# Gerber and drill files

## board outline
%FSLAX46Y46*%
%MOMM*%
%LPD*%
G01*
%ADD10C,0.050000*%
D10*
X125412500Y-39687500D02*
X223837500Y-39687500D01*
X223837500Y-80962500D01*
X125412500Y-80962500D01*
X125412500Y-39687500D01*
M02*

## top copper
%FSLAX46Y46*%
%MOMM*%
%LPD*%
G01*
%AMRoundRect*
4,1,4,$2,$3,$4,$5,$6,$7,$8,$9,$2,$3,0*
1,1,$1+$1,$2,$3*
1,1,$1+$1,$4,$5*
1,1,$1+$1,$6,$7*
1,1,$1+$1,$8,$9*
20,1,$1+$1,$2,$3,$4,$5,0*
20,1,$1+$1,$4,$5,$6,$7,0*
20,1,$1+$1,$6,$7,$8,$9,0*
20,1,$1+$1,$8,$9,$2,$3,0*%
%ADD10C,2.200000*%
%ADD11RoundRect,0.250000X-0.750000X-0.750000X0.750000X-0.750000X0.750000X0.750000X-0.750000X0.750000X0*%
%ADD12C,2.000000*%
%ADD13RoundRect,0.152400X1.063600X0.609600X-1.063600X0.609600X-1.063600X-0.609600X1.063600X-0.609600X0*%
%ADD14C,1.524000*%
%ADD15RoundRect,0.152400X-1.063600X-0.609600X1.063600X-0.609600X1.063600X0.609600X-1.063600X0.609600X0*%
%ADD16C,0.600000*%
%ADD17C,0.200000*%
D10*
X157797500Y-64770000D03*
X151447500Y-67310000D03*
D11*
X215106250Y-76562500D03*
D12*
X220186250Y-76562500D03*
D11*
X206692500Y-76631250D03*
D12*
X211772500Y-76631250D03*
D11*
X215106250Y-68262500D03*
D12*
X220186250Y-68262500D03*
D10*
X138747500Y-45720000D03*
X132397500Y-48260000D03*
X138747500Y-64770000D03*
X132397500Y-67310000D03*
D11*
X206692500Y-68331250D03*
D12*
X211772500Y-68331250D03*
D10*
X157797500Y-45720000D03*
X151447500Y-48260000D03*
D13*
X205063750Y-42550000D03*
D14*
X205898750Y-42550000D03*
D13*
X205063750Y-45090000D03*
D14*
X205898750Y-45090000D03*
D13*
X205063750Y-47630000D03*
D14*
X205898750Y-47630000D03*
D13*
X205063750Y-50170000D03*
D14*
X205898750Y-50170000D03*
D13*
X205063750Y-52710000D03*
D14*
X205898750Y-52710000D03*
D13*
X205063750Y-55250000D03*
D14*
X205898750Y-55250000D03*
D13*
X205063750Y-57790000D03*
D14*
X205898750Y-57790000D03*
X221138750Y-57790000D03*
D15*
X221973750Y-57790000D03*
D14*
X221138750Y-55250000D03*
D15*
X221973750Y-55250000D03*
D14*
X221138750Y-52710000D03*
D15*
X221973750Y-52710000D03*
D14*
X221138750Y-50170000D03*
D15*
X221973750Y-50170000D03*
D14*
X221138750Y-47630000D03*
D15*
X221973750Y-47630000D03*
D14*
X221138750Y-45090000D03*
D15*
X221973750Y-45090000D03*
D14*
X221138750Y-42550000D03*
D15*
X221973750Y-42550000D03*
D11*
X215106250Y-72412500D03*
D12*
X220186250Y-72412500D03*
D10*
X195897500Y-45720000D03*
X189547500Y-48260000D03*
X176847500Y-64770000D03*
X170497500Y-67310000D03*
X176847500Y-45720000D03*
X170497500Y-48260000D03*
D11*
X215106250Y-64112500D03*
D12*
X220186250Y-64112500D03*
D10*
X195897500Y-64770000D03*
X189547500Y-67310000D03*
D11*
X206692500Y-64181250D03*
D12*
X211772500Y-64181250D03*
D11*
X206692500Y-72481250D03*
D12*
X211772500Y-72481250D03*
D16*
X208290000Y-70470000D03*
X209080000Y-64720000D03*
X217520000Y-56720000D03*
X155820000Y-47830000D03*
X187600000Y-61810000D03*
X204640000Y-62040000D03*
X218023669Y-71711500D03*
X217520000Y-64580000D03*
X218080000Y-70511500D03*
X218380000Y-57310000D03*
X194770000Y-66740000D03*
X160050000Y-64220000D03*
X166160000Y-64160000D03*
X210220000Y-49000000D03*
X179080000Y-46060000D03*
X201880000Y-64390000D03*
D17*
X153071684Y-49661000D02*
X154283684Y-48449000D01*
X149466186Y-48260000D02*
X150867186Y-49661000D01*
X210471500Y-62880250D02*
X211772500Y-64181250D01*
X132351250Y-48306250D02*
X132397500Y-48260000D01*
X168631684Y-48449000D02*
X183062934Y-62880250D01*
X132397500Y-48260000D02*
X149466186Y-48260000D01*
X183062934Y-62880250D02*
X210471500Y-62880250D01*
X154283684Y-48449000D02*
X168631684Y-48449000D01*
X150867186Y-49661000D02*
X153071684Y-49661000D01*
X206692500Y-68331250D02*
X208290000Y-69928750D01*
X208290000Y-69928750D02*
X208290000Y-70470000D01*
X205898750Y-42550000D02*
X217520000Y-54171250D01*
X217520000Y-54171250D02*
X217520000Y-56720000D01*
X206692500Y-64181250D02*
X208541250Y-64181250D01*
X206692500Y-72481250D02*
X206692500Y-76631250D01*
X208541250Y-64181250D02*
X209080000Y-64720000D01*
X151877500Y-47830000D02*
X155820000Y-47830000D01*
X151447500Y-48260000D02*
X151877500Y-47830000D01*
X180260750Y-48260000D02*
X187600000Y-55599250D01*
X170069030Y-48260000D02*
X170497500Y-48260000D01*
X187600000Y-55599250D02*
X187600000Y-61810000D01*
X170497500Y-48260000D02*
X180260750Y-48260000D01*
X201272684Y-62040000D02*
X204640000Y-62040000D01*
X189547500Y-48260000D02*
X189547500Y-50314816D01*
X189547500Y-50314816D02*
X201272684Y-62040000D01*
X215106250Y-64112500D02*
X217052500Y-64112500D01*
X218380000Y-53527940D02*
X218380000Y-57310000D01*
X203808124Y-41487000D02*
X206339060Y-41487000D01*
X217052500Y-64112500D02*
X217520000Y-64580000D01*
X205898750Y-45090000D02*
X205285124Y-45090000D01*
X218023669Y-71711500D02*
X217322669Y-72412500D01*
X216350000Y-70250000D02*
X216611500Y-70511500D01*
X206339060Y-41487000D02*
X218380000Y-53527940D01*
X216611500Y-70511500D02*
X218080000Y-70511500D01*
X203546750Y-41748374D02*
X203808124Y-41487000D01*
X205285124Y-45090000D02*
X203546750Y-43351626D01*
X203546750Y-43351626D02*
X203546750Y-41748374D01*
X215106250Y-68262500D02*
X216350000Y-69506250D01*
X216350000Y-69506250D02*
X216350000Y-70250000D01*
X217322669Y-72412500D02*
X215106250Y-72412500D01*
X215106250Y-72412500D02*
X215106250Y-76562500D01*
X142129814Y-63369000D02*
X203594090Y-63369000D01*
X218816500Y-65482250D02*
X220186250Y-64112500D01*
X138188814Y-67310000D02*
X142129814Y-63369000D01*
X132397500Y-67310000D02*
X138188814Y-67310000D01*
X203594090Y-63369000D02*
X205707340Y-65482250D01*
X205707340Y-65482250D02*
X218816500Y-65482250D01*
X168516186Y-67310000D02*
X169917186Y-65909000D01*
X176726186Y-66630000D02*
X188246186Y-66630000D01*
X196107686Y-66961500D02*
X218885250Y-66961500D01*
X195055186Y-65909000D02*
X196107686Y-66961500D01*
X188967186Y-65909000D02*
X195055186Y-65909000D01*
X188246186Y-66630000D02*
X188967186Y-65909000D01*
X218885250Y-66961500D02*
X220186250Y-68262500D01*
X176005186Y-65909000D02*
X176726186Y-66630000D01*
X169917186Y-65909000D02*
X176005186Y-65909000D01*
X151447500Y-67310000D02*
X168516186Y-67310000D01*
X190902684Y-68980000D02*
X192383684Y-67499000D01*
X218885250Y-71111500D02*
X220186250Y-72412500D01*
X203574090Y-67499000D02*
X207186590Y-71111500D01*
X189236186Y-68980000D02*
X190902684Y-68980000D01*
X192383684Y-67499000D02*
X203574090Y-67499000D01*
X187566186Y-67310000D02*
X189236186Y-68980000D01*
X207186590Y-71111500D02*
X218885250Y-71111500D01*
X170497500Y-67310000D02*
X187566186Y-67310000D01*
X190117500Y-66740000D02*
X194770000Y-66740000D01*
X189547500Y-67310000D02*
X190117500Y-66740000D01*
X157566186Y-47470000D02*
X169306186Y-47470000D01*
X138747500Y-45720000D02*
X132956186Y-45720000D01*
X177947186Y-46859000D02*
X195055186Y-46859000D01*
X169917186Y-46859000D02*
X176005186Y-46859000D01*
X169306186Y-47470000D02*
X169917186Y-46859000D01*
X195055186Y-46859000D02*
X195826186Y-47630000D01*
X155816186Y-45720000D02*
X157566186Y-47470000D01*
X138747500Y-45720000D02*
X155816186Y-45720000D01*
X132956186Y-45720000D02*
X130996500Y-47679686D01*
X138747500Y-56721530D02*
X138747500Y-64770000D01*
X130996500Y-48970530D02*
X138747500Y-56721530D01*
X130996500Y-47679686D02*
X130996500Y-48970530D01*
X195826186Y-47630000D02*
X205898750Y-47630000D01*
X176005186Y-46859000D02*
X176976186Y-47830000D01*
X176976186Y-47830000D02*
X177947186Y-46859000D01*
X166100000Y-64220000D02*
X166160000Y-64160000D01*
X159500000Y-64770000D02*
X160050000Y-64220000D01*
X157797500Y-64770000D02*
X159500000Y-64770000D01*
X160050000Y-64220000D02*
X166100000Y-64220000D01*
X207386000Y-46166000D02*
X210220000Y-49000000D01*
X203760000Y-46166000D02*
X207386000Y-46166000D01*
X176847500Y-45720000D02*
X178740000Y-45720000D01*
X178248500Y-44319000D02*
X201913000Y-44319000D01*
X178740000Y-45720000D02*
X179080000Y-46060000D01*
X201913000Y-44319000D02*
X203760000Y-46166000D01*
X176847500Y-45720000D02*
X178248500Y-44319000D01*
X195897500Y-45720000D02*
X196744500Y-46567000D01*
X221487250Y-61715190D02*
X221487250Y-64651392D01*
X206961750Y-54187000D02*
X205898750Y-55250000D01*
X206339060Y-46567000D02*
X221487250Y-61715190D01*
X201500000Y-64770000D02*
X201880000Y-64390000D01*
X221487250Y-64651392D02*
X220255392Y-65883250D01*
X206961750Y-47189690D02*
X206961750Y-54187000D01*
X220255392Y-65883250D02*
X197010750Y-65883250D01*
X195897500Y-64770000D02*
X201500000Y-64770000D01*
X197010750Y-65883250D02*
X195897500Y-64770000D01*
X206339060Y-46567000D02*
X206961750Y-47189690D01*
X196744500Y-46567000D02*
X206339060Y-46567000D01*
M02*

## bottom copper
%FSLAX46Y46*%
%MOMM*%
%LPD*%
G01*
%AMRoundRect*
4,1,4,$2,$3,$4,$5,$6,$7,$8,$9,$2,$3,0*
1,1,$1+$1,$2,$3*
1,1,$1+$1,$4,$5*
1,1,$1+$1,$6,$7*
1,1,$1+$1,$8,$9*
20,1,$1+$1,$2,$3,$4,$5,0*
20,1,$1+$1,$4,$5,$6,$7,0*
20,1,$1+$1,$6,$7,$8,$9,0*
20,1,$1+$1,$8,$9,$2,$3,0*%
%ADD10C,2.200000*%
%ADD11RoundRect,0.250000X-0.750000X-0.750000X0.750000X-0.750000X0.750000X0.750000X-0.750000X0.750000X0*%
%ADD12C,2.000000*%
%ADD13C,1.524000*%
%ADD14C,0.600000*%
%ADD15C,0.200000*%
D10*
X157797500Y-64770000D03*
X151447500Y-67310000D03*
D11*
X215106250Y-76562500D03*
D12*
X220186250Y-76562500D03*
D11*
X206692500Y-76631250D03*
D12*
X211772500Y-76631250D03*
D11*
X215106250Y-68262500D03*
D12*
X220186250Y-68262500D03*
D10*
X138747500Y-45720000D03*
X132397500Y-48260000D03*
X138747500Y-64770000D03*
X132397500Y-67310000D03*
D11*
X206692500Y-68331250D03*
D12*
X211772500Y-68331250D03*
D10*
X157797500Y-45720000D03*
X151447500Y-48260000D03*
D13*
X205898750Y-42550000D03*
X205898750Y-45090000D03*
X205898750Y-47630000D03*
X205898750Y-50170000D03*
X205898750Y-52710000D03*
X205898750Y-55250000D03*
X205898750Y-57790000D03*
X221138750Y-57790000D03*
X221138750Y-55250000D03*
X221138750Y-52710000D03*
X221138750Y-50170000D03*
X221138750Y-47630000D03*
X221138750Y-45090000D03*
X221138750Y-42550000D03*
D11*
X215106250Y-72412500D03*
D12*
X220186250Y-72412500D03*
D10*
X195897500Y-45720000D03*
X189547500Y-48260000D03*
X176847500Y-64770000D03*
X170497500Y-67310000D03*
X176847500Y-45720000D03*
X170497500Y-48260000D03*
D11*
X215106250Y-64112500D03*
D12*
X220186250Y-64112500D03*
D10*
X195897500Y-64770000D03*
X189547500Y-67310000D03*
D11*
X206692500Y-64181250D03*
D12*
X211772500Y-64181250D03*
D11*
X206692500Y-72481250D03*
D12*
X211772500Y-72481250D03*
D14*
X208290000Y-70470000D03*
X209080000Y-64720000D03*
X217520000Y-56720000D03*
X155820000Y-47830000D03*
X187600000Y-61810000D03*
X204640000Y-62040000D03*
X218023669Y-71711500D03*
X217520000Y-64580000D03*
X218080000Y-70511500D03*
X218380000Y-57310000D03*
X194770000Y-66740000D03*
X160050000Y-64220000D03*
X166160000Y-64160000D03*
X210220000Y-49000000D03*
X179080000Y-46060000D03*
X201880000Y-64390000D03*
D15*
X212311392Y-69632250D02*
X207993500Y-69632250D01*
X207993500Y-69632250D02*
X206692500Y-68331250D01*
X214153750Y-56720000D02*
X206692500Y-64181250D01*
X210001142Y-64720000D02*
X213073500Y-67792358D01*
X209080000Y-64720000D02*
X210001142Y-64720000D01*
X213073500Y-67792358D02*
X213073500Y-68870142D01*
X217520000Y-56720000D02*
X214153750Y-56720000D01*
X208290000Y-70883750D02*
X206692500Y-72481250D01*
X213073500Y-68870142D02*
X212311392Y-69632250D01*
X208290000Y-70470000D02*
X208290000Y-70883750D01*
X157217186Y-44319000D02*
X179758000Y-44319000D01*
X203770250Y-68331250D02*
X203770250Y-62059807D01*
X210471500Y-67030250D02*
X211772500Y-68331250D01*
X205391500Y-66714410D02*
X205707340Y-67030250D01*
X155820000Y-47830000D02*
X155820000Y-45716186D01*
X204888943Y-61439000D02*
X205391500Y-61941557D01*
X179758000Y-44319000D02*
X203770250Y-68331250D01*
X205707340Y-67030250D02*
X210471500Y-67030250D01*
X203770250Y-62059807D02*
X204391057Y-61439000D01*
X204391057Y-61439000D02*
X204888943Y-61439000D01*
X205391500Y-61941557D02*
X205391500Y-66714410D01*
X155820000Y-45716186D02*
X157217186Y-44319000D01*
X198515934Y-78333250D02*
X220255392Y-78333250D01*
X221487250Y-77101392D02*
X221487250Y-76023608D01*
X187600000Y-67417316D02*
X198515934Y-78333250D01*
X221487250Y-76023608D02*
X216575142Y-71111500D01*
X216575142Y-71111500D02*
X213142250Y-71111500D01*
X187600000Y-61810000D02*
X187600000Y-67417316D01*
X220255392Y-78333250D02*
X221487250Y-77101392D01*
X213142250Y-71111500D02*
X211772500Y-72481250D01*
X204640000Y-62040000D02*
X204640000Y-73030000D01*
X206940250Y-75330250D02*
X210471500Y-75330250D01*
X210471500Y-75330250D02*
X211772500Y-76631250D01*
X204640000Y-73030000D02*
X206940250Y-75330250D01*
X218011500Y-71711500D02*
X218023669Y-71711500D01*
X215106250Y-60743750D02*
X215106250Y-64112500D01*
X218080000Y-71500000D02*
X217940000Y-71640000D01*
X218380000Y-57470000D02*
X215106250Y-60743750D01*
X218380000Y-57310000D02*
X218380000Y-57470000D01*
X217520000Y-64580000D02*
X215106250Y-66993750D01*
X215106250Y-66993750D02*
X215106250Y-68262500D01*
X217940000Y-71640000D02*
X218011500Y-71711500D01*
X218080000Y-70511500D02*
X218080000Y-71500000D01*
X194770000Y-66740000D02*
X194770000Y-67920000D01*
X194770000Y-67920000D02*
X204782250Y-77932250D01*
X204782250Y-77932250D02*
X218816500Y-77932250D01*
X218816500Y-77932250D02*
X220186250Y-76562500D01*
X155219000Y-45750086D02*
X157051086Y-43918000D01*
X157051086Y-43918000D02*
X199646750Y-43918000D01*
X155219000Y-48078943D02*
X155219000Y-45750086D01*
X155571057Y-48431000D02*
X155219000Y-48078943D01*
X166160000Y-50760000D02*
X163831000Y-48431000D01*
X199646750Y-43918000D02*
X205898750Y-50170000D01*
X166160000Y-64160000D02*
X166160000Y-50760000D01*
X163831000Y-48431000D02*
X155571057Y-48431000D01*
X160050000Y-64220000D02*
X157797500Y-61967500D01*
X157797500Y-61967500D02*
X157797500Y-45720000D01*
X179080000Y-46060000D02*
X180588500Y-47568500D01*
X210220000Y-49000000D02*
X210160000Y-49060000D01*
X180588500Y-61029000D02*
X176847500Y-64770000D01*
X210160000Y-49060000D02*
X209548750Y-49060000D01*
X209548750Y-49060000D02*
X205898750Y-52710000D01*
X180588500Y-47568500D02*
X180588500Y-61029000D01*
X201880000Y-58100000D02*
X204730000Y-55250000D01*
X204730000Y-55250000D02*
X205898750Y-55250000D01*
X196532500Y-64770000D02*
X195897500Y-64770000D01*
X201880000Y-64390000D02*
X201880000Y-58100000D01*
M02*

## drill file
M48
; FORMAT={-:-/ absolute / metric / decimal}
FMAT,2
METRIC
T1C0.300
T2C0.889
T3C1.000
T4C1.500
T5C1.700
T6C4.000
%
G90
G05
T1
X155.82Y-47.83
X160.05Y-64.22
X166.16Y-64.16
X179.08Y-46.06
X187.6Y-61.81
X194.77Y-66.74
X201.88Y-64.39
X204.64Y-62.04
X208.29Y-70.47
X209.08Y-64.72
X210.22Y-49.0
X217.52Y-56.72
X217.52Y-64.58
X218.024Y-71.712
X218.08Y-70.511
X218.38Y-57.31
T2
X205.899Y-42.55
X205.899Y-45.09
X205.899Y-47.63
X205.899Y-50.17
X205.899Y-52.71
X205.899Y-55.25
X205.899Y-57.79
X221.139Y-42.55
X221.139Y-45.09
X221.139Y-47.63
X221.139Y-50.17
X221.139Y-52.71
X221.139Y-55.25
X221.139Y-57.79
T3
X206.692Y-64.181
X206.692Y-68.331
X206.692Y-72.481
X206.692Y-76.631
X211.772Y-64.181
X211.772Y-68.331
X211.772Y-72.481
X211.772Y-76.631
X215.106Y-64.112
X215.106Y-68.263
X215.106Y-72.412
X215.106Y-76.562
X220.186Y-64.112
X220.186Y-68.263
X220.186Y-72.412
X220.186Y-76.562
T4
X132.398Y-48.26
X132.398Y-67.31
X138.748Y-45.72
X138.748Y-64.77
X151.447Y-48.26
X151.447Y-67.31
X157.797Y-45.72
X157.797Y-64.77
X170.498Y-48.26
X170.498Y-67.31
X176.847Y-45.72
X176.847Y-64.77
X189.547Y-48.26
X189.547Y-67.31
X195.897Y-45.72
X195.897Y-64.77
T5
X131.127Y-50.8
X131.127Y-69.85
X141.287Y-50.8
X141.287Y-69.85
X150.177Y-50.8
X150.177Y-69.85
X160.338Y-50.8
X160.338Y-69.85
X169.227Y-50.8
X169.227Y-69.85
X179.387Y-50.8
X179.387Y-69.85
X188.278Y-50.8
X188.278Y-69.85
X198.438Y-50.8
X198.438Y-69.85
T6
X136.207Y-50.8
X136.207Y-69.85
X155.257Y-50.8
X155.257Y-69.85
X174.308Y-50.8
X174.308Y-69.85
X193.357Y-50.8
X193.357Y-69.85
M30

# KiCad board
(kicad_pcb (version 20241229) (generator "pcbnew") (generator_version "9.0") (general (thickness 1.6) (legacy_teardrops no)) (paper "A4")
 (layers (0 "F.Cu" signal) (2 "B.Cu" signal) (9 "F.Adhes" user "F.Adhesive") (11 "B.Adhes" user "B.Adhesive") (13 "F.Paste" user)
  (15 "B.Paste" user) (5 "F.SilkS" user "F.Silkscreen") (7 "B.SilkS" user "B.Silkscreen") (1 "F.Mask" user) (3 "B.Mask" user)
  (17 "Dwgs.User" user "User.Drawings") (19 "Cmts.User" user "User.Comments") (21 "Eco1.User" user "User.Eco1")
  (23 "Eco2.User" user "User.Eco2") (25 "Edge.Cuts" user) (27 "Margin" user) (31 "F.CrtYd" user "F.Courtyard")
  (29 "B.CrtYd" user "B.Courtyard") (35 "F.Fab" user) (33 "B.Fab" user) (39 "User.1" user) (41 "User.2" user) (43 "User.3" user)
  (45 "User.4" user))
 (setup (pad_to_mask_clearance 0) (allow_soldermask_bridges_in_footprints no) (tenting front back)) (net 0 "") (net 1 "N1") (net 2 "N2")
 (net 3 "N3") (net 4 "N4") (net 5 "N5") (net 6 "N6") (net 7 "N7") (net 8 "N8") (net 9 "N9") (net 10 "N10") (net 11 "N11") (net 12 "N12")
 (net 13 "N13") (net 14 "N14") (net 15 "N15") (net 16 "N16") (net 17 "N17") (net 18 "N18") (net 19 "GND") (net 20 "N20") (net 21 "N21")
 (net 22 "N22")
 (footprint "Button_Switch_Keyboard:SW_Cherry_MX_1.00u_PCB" (layer "F.Cu") (at 157.7975 64.77)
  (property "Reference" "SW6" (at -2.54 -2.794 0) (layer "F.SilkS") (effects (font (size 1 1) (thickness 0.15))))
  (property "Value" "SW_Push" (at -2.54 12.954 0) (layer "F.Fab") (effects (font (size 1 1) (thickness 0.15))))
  (pad "" np_thru_hole circle (at -7.62 5.08) (size 1.7 1.7) (drill 1.7) (layers "*.Cu" "*.Mask"))
  (pad "" np_thru_hole circle (at -2.54 5.08) (size 4 4) (drill 4) (layers "*.Cu" "*.Mask"))
  (pad "" np_thru_hole circle (at 2.54 5.08) (size 1.7 1.7) (drill 1.7) (layers "*.Cu" "*.Mask"))
  (pad "1" thru_hole circle (at 0 0) (size 2.2 2.2) (drill 1.5) (layers "*.Cu" "*.Mask") (remove_unused_layers no) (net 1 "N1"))
  (pad "2" thru_hole circle (at -6.35 2.54) (size 2.2 2.2) (drill 1.5) (layers "*.Cu" "*.Mask") (remove_unused_layers no) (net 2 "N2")))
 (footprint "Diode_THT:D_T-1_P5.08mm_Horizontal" (layer "F.Cu") (at 215.10625 76.5625)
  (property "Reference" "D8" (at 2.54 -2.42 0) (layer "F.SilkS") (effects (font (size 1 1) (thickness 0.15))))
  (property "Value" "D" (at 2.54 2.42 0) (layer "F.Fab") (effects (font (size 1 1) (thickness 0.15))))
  (pad "1" thru_hole roundrect (at 0 0) (size 2 2) (drill 1) (layers "*.Cu" "*.Mask") (remove_unused_layers no) (roundrect_rratio 0.125)
   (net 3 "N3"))
  (pad "2" thru_hole circle (at 5.08 0) (size 2 2) (drill 1) (layers "*.Cu" "*.Mask") (remove_unused_layers no) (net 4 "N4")))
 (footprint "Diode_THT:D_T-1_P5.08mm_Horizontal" (layer "F.Cu") (at 206.6925 76.63125)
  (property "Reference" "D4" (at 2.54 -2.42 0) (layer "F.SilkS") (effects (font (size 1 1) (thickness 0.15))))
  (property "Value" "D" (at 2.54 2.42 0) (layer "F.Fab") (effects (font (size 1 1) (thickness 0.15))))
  (pad "1" thru_hole roundrect (at 0 0) (size 2 2) (drill 1) (layers "*.Cu" "*.Mask") (remove_unused_layers no) (roundrect_rratio 0.125)
   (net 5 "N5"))
  (pad "2" thru_hole circle (at 5.08 0) (size 2 2) (drill 1) (layers "*.Cu" "*.Mask") (remove_unused_layers no) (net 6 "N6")))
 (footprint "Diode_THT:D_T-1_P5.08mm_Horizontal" (layer "F.Cu") (at 215.10625 68.2625)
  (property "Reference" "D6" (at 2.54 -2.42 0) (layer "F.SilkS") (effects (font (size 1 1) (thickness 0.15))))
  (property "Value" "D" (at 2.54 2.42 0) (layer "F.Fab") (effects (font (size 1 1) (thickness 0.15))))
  (pad "1" thru_hole roundrect (at 0 0) (size 2 2) (drill 1) (layers "*.Cu" "*.Mask") (remove_unused_layers no) (roundrect_rratio 0.125)
   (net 3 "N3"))
  (pad "2" thru_hole circle (at 5.08 0) (size 2 2) (drill 1) (layers "*.Cu" "*.Mask") (remove_unused_layers no) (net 2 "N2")))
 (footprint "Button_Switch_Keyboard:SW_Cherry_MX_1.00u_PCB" (layer "F.Cu") (at 138.7475 45.72)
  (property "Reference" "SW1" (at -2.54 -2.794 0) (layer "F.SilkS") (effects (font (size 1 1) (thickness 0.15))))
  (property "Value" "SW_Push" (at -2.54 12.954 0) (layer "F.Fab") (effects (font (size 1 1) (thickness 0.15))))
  (pad "" np_thru_hole circle (at -7.62 5.08) (size 1.7 1.7) (drill 1.7) (layers "*.Cu" "*.Mask"))
  (pad "" np_thru_hole circle (at -2.54 5.08) (size 4 4) (drill 4) (layers "*.Cu" "*.Mask"))
  (pad "" np_thru_hole circle (at 2.54 5.08) (size 1.7 1.7) (drill 1.7) (layers "*.Cu" "*.Mask"))
  (pad "1" thru_hole circle (at 0 0) (size 2.2 2.2) (drill 1.5) (layers "*.Cu" "*.Mask") (remove_unused_layers no) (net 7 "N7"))
  (pad "2" thru_hole circle (at -6.35 2.54) (size 2.2 2.2) (drill 1.5) (layers "*.Cu" "*.Mask") (remove_unused_layers no) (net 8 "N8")))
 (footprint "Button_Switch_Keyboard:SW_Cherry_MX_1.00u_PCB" (layer "F.Cu") (at 138.7475 64.77)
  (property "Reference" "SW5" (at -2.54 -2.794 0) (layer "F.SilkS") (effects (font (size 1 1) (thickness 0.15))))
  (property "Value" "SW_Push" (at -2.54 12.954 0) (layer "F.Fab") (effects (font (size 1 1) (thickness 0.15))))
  (pad "" np_thru_hole circle (at -7.62 5.08) (size 1.7 1.7) (drill 1.7) (layers "*.Cu" "*.Mask"))
  (pad "" np_thru_hole circle (at -2.54 5.08) (size 4 4) (drill 4) (layers "*.Cu" "*.Mask"))
  (pad "" np_thru_hole circle (at 2.54 5.08) (size 1.7 1.7) (drill 1.7) (layers "*.Cu" "*.Mask"))
  (pad "1" thru_hole circle (at 0 0) (size 2.2 2.2) (drill 1.5) (layers "*.Cu" "*.Mask") (remove_unused_layers no) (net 7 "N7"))
  (pad "2" thru_hole circle (at -6.35 2.54) (size 2.2 2.2) (drill 1.5) (layers "*.Cu" "*.Mask") (remove_unused_layers no) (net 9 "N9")))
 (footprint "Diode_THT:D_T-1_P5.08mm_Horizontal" (layer "F.Cu") (at 206.6925 68.33125)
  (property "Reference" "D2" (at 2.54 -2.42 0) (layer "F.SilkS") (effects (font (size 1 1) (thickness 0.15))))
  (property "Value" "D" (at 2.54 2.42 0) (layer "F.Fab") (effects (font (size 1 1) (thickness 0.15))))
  (pad "1" thru_hole roundrect (at 0 0) (size 2 2) (drill 1) (layers "*.Cu" "*.Mask") (remove_unused_layers no) (roundrect_rratio 0.125)
   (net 5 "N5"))
  (pad "2" thru_hole circle (at 5.08 0) (size 2 2) (drill 1) (layers "*.Cu" "*.Mask") (remove_unused_layers no) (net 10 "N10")))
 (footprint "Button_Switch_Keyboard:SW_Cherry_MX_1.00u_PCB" (layer "F.Cu") (at 157.7975 45.72)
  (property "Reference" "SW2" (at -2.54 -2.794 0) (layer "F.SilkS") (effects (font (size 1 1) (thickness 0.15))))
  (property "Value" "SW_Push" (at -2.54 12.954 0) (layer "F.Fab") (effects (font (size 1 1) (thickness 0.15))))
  (pad "" np_thru_hole circle (at -7.62 5.08) (size 1.7 1.7) (drill 1.7) (layers "*.Cu" "*.Mask"))
  (pad "" np_thru_hole circle (at -2.54 5.08) (size 4 4) (drill 4) (layers "*.Cu" "*.Mask"))
  (pad "" np_thru_hole circle (at 2.54 5.08) (size 1.7 1.7) (drill 1.7) (layers "*.Cu" "*.Mask"))
  (pad "1" thru_hole circle (at 0 0) (size 2.2 2.2) (drill 1.5) (layers "*.Cu" "*.Mask") (remove_unused_layers no) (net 1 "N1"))
  (pad "2" thru_hole circle (at -6.35 2.54) (size 2.2 2.2) (drill 1.5) (layers "*.Cu" "*.Mask") (remove_unused_layers no) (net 10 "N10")))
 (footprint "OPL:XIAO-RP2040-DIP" (layer "F.Cu") (at 213.51875 50.17)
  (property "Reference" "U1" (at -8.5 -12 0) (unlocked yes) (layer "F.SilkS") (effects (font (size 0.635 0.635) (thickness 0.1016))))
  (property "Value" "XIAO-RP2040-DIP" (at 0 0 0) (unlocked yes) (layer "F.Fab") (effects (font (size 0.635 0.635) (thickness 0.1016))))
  (pad "1" smd roundrect (at -8.455 -7.62 180) (size 2.432 1.524) (layers "F.Cu" "F.Mask") (roundrect_rratio 0.1) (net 5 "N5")
   (thermal_bridge_angle 45))
  (pad "1" thru_hole circle (at -7.62 -7.62 180) (size 1.524 1.524) (drill 0.889) (layers "*.Cu" "*.Mask") (remove_unused_layers no)
   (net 5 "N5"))
  (pad "2" smd roundrect (at -8.455 -5.08 180) (size 2.432 1.524) (layers "F.Cu" "F.Mask") (roundrect_rratio 0.1) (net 3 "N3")
   (thermal_bridge_angle 45))
  (pad "2" thru_hole circle (at -7.62 -5.08 180) (size 1.524 1.524) (drill 0.889) (layers "*.Cu" "*.Mask") (remove_unused_layers no)
   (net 3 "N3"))
  (pad "3" smd roundrect (at -8.455 -2.54 180) (size 2.432 1.524) (layers "F.Cu" "F.Mask") (roundrect_rratio 0.1) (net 7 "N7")
   (thermal_bridge_angle 45))
  (pad "3" thru_hole circle (at -7.62 -2.54 180) (size 1.524 1.524) (drill 0.889) (layers "*.Cu" "*.Mask") (remove_unused_layers no)
   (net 7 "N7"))
  (pad "4" smd roundrect (at -8.455 0 180) (size 2.432 1.524) (layers "F.Cu" "F.Mask") (roundrect_rratio 0.1) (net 1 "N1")
   (thermal_bridge_angle 45))
  (pad "4" thru_hole circle (at -7.62 0 180) (size 1.524 1.524) (drill 0.889) (layers "*.Cu" "*.Mask") (remove_unused_layers no)
   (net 1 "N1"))
  (pad "5" smd roundrect (at -8.455 2.54 180) (size 2.432 1.524) (layers "F.Cu" "F.Mask") (roundrect_rratio 0.1) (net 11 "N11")
   (thermal_bridge_angle 45))
  (pad "5" thru_hole circle (at -7.62 2.54 180) (size 1.524 1.524) (drill 0.889) (layers "*.Cu" "*.Mask") (remove_unused_layers no)
   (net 11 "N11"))
  (pad "6" smd roundrect (at -8.455 5.08 180) (size 2.432 1.524) (layers "F.Cu" "F.Mask") (roundrect_rratio 0.1) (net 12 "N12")
   (thermal_bridge_angle 45))
  (pad "6" thru_hole circle (at -7.62 5.08 180) (size 1.524 1.524) (drill 0.889) (layers "*.Cu" "*.Mask") (remove_unused_layers no)
   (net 12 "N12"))
  (pad "7" smd roundrect (at -8.455 7.62 180) (size 2.432 1.524) (layers "F.Cu" "F.Mask") (roundrect_rratio 0.1) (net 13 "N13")
   (thermal_bridge_angle 45))
  (pad "7" thru_hole circle (at -7.62 7.62 180) (size 1.524 1.524) (drill 0.889) (layers "*.Cu" "*.Mask") (remove_unused_layers no)
   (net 13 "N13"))
  (pad "8" thru_hole circle (at 7.62 7.62) (size 1.524 1.524) (drill 0.889) (layers "*.Cu" "*.Mask") (remove_unused_layers no)
   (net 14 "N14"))
  (pad "8" smd roundrect (at 8.455 7.62) (size 2.432 1.524) (layers "F.Cu" "F.Mask") (roundrect_rratio 0.1) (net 14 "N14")
   (thermal_bridge_angle 45))
  (pad "9" thru_hole circle (at 7.62 5.08) (size 1.524 1.524) (drill 0.889) (layers "*.Cu" "*.Mask") (remove_unused_layers no)
   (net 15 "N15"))
  (pad "9" smd roundrect (at 8.455 5.08) (size 2.432 1.524) (layers "F.Cu" "F.Mask") (roundrect_rratio 0.1) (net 15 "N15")
   (thermal_bridge_angle 45))
  (pad "10" thru_hole circle (at 7.62 2.54) (size 1.524 1.524) (drill 0.889) (layers "*.Cu" "*.Mask") (remove_unused_layers no)
   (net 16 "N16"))
  (pad "10" smd roundrect (at 8.455 2.54) (size 2.432 1.524) (layers "F.Cu" "F.Mask") (roundrect_rratio 0.1) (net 16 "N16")
   (thermal_bridge_angle 45))
  (pad "11" thru_hole circle (at 7.62 0) (size 1.524 1.524) (drill 0.889) (layers "*.Cu" "*.Mask") (remove_unused_layers no) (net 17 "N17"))
  (pad "11" smd roundrect (at 8.455 0) (size 2.432 1.524) (layers "F.Cu" "F.Mask") (roundrect_rratio 0.1) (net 17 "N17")
   (thermal_bridge_angle 45))
  (pad "12" thru_hole circle (at 7.62 -2.54) (size 1.524 1.524) (drill 0.889) (layers "*.Cu" "*.Mask") (remove_unused_layers no)
   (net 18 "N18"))
  (pad "12" smd roundrect (at 8.455 -2.54) (size 2.432 1.524) (layers "F.Cu" "F.Mask") (roundrect_rratio 0.1) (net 18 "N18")
   (thermal_bridge_angle 45))
  (pad "13" thru_hole circle (at 7.62 -5.08) (size 1.524 1.524) (drill 0.889) (layers "*.Cu" "*.Mask") (remove_unused_layers no)
   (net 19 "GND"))
  (pad "13" smd roundrect (at 8.455 -5.08) (size 2.432 1.524) (layers "F.Cu" "F.Mask") (roundrect_rratio 0.1) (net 19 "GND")
   (thermal_bridge_angle 45))
  (pad "14" thru_hole circle (at 7.62 -7.62) (size 1.524 1.524) (drill 0.889) (layers "*.Cu" "*.Mask") (remove_unused_layers no)
   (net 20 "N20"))
  (pad "14" smd roundrect (at 8.455 -7.62) (size 2.432 1.524) (layers "F.Cu" "F.Mask") (roundrect_rratio 0.1) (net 20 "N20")
   (thermal_bridge_angle 45)))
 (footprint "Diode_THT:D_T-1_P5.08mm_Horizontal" (layer "F.Cu") (at 215.10625 72.4125)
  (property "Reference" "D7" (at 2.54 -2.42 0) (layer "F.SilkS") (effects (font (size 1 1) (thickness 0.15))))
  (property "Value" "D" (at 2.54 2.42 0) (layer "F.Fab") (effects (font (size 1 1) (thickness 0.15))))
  (pad "1" thru_hole roundrect (at 0 0) (size 2 2) (drill 1) (layers "*.Cu" "*.Mask") (remove_unused_layers no) (roundrect_rratio 0.125)
   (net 3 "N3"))
  (pad "2" thru_hole circle (at 5.08 0) (size 2 2) (drill 1) (layers "*.Cu" "*.Mask") (remove_unused_layers no) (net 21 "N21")))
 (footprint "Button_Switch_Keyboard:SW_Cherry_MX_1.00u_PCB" (layer "F.Cu") (at 195.8975 45.72)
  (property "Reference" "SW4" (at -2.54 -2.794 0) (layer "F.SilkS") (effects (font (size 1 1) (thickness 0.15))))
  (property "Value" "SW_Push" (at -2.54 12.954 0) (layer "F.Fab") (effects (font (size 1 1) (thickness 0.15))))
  (pad "" np_thru_hole circle (at -7.62 5.08) (size 1.7 1.7) (drill 1.7) (layers "*.Cu" "*.Mask"))
  (pad "" np_thru_hole circle (at -2.54 5.08) (size 4 4) (drill 4) (layers "*.Cu" "*.Mask"))
  (pad "" np_thru_hole circle (at 2.54 5.08) (size 1.7 1.7) (drill 1.7) (layers "*.Cu" "*.Mask"))
  (pad "1" thru_hole circle (at 0 0) (size 2.2 2.2) (drill 1.5) (layers "*.Cu" "*.Mask") (remove_unused_layers no) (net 12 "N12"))
  (pad "2" thru_hole circle (at -6.35 2.54) (size 2.2 2.2) (drill 1.5) (layers "*.Cu" "*.Mask") (remove_unused_layers no) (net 6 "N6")))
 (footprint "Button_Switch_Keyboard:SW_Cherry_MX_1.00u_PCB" (layer "F.Cu") (at 176.8475 64.77)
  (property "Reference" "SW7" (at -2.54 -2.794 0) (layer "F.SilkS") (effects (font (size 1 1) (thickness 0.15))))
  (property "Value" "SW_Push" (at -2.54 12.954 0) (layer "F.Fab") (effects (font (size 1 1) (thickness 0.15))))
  (pad "" np_thru_hole circle (at -7.62 5.08) (size 1.7 1.7) (drill 1.7) (layers "*.Cu" "*.Mask"))
  (pad "" np_thru_hole circle (at -2.54 5.08) (size 4 4) (drill 4) (layers "*.Cu" "*.Mask"))
  (pad "" np_thru_hole circle (at 2.54 5.08) (size 1.7 1.7) (drill 1.7) (layers "*.Cu" "*.Mask"))
  (pad "1" thru_hole circle (at 0 0) (size 2.2 2.2) (drill 1.5) (layers "*.Cu" "*.Mask") (remove_unused_layers no) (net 11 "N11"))
  (pad "2" thru_hole circle (at -6.35 2.54) (size 2.2 2.2) (drill 1.5) (layers "*.Cu" "*.Mask") (remove_unused_layers no) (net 21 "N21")))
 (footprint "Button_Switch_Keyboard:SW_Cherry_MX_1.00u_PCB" (layer "F.Cu") (at 176.8475 45.72)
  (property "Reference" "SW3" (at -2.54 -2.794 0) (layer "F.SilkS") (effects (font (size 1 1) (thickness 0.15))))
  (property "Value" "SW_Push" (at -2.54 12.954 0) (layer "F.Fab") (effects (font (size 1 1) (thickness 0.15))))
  (pad "" np_thru_hole circle (at -7.62 5.08) (size 1.7 1.7) (drill 1.7) (layers "*.Cu" "*.Mask"))
  (pad "" np_thru_hole circle (at -2.54 5.08) (size 4 4) (drill 4) (layers "*.Cu" "*.Mask"))
  (pad "" np_thru_hole circle (at 2.54 5.08) (size 1.7 1.7) (drill 1.7) (layers "*.Cu" "*.Mask"))
  (pad "1" thru_hole circle (at 0 0) (size 2.2 2.2) (drill 1.5) (layers "*.Cu" "*.Mask") (remove_unused_layers no) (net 11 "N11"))
  (pad "2" thru_hole circle (at -6.35 2.54) (size 2.2 2.2) (drill 1.5) (layers "*.Cu" "*.Mask") (remove_unused_layers no) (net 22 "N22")))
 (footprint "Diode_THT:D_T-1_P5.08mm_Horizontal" (layer "F.Cu") (at 215.10625 64.1125)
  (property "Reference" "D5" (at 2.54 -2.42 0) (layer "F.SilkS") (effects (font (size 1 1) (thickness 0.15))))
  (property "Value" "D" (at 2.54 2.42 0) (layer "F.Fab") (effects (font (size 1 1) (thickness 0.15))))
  (pad "1" thru_hole roundrect (at 0 0) (size 2 2) (drill 1) (layers "*.Cu" "*.Mask") (remove_unused_layers no) (roundrect_rratio 0.125)
   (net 3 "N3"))
  (pad "2" thru_hole circle (at 5.08 0) (size 2 2) (drill 1) (layers "*.Cu" "*.Mask") (remove_unused_layers no) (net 9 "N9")))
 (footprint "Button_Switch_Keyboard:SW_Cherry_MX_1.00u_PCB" (layer "F.Cu") (at 195.8975 64.77)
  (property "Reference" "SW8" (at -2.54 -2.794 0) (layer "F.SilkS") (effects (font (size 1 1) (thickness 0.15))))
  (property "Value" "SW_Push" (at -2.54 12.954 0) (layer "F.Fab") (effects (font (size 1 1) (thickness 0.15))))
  (pad "" np_thru_hole circle (at -7.62 5.08) (size 1.7 1.7) (drill 1.7) (layers "*.Cu" "*.Mask"))
  (pad "" np_thru_hole circle (at -2.54 5.08) (size 4 4) (drill 4) (layers "*.Cu" "*.Mask"))
  (pad "" np_thru_hole circle (at 2.54 5.08) (size 1.7 1.7) (drill 1.7) (layers "*.Cu" "*.Mask"))
  (pad "1" thru_hole circle (at 0 0) (size 2.2 2.2) (drill 1.5) (layers "*.Cu" "*.Mask") (remove_unused_layers no) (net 12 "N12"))
  (pad "2" thru_hole circle (at -6.35 2.54) (size 2.2 2.2) (drill 1.5) (layers "*.Cu" "*.Mask") (remove_unused_layers no) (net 4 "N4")))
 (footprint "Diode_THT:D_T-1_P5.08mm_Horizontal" (layer "F.Cu") (at 206.6925 64.18125)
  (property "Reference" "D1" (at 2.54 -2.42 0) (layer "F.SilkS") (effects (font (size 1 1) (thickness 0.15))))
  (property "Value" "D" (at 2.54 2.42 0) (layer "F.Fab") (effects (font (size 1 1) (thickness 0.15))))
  (pad "1" thru_hole roundrect (at 0 0) (size 2 2) (drill 1) (layers "*.Cu" "*.Mask") (remove_unused_layers no) (roundrect_rratio 0.125)
   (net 5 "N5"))
  (pad "2" thru_hole circle (at 5.08 0) (size 2 2) (drill 1) (layers "*.Cu" "*.Mask") (remove_unused_layers no) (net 8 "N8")))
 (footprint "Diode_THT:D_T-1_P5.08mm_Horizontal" (layer "F.Cu") (at 206.6925 72.48125)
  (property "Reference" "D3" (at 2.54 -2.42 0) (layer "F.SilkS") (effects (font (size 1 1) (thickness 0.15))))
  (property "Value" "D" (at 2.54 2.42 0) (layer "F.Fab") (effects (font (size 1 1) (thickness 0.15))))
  (pad "1" thru_hole roundrect (at 0 0) (size 2 2) (drill 1) (layers "*.Cu" "*.Mask") (remove_unused_layers no) (roundrect_rratio 0.125)
   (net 5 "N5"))
  (pad "2" thru_hole circle (at 5.08 0) (size 2 2) (drill 1) (layers "*.Cu" "*.Mask") (remove_unused_layers no) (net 22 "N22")))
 (gr_rect (start 125.4125 39.6875) (end 223.8375 80.9625) (stroke (width 0.05) (type default)) (fill no) (layer "Edge.Cuts"))
 (segment (start 153.071684 49.661) (end 154.283684 48.449) (width 0.2) (layer "F.Cu") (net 8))
 (segment (start 149.466186 48.26) (end 150.867186 49.661) (width 0.2) (layer "F.Cu") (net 8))
 (segment (start 210.4715 62.88025) (end 211.7725 64.18125) (width 0.2) (layer "F.Cu") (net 8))
 (segment (start 132.35125 48.30625) (end 132.3975 48.26) (width 0.2) (layer "F.Cu") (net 8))
 (segment (start 168.631684 48.449) (end 183.062934 62.88025) (width 0.2) (layer "F.Cu") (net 8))
 (segment (start 132.3975 48.26) (end 149.466186 48.26) (width 0.2) (layer "F.Cu") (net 8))
 (segment (start 183.062934 62.88025) (end 210.4715 62.88025) (width 0.2) (layer "F.Cu") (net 8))
 (segment (start 154.283684 48.449) (end 168.631684 48.449) (width 0.2) (layer "F.Cu") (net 8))
 (segment (start 150.867186 49.661) (end 153.071684 49.661) (width 0.2) (layer "F.Cu") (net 8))
 (segment (start 206.6925 68.33125) (end 208.29 69.92875) (width 0.2) (layer "F.Cu") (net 5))
 (segment (start 208.29 69.92875) (end 208.29 70.47) (width 0.2) (layer "F.Cu") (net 5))
 (segment (start 205.89875 42.55) (end 217.52 54.17125) (width 0.2) (layer "F.Cu") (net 5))
 (segment (start 217.52 54.17125) (end 217.52 56.72) (width 0.2) (layer "F.Cu") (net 5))
 (segment (start 206.6925 64.18125) (end 208.54125 64.18125) (width 0.2) (layer "F.Cu") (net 5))
 (segment (start 206.6925 72.48125) (end 206.6925 76.63125) (width 0.2) (layer "F.Cu") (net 5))
 (segment (start 208.54125 64.18125) (end 209.08 64.72) (width 0.2) (layer "F.Cu") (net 5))
 (via (at 208.29 70.47) (size 0.6) (drill 0.3) (layers "F.Cu" "B.Cu") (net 5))
 (via (at 209.08 64.72) (size 0.6) (drill 0.3) (layers "F.Cu" "B.Cu") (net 5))
 (via (at 217.52 56.72) (size 0.6) (drill 0.3) (layers "F.Cu" "B.Cu") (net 5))
 (segment (start 212.311392 69.63225) (end 207.9935 69.63225) (width 0.2) (layer "B.Cu") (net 5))
 (segment (start 207.9935 69.63225) (end 206.6925 68.33125) (width 0.2) (layer "B.Cu") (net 5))
 (segment (start 214.15375 56.72) (end 206.6925 64.18125) (width 0.2) (layer "B.Cu") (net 5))
 (segment (start 210.001142 64.72) (end 213.0735 67.792358) (width 0.2) (layer "B.Cu") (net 5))
 (segment (start 209.08 64.72) (end 210.001142 64.72) (width 0.2) (layer "B.Cu") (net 5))
 (segment (start 213.0735 67.792358) (end 213.0735 68.870142) (width 0.2) (layer "B.Cu") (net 5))
 (segment (start 217.52 56.72) (end 214.15375 56.72) (width 0.2) (layer "B.Cu") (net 5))
 (segment (start 208.29 70.88375) (end 206.6925 72.48125) (width 0.2) (layer "B.Cu") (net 5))
 (segment (start 213.0735 68.870142) (end 212.311392 69.63225) (width 0.2) (layer "B.Cu") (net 5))
 (segment (start 208.29 70.47) (end 208.29 70.88375) (width 0.2) (layer "B.Cu") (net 5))
 (segment (start 151.8775 47.83) (end 155.82 47.83) (width 0.2) (layer "F.Cu") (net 10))
 (segment (start 151.4475 48.26) (end 151.8775 47.83) (width 0.2) (layer "F.Cu") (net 10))
 (via (at 155.82 47.83) (size 0.6) (drill 0.3) (layers "F.Cu" "B.Cu") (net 10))
 (segment (start 157.217186 44.319) (end 179.758 44.319) (width 0.2) (layer "B.Cu") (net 10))
 (segment (start 203.77025 68.33125) (end 203.77025 62.059807) (width 0.2) (layer "B.Cu") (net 10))
 (segment (start 210.4715 67.03025) (end 211.7725 68.33125) (width 0.2) (layer "B.Cu") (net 10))
 (segment (start 205.3915 66.71441) (end 205.70734 67.03025) (width 0.2) (layer "B.Cu") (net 10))
 (segment (start 155.82 47.83) (end 155.82 45.716186) (width 0.2) (layer "B.Cu") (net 10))
 (segment (start 204.888943 61.439) (end 205.3915 61.941557) (width 0.2) (layer "B.Cu") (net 10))
 (segment (start 179.758 44.319) (end 203.77025 68.33125) (width 0.2) (layer "B.Cu") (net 10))
 (segment (start 205.70734 67.03025) (end 210.4715 67.03025) (width 0.2) (layer "B.Cu") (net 10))
 (segment (start 203.77025 62.059807) (end 204.391057 61.439) (width 0.2) (layer "B.Cu") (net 10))
 (segment (start 204.391057 61.439) (end 204.888943 61.439) (width 0.2) (layer "B.Cu") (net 10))
 (segment (start 205.3915 61.941557) (end 205.3915 66.71441) (width 0.2) (layer "B.Cu") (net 10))
 (segment (start 155.82 45.716186) (end 157.217186 44.319) (width 0.2) (layer "B.Cu") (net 10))
 (segment (start 180.26075 48.26) (end 187.6 55.59925) (width 0.2) (layer "F.Cu") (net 22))
 (segment (start 170.06903 48.26) (end 170.4975 48.26) (width 0.2) (layer "F.Cu") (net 22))
 (segment (start 187.6 55.59925) (end 187.6 61.81) (width 0.2) (layer "F.Cu") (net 22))
 (segment (start 170.4975 48.26) (end 180.26075 48.26) (width 0.2) (layer "F.Cu") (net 22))
 (via (at 187.6 61.81) (size 0.6) (drill 0.3) (layers "F.Cu" "B.Cu") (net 22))
 (segment (start 198.515934 78.33325) (end 220.255392 78.33325) (width 0.2) (layer "B.Cu") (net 22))
 (segment (start 221.48725 77.101392) (end 221.48725 76.023608) (width 0.2) (layer "B.Cu") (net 22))
 (segment (start 187.6 67.417316) (end 198.515934 78.33325) (width 0.2) (layer "B.Cu") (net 22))
 (segment (start 221.48725 76.023608) (end 216.575142 71.1115) (width 0.2) (layer "B.Cu") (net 22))
 (segment (start 216.575142 71.1115) (end 213.14225 71.1115) (width 0.2) (layer "B.Cu") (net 22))
 (segment (start 187.6 61.81) (end 187.6 67.417316) (width 0.2) (layer "B.Cu") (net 22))
 (segment (start 220.255392 78.33325) (end 221.48725 77.101392) (width 0.2) (layer "B.Cu") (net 22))
 (segment (start 213.14225 71.1115) (end 211.7725 72.48125) (width 0.2) (layer "B.Cu") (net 22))
 (segment (start 201.272684 62.04) (end 204.64 62.04) (width 0.2) (layer "F.Cu") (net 6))
 (segment (start 189.5475 48.26) (end 189.5475 50.314816) (width 0.2) (layer "F.Cu") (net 6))
 (segment (start 189.5475 50.314816) (end 201.272684 62.04) (width 0.2) (layer "F.Cu") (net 6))
 (via (at 204.64 62.04) (size 0.6) (drill 0.3) (layers "F.Cu" "B.Cu") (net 6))
 (segment (start 204.64 62.04) (end 204.64 73.03) (width 0.2) (layer "B.Cu") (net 6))
 (segment (start 206.94025 75.33025) (end 210.4715 75.33025) (width 0.2) (layer "B.Cu") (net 6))
 (segment (start 210.4715 75.33025) (end 211.7725 76.63125) (width 0.2) (layer "B.Cu") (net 6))
 (segment (start 204.64 73.03) (end 206.94025 75.33025) (width 0.2) (layer "B.Cu") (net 6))
 (segment (start 215.10625 64.1125) (end 217.0525 64.1125) (width 0.2) (layer "F.Cu") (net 3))
 (segment (start 218.38 53.52794) (end 218.38 57.31) (width 0.2) (layer "F.Cu") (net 3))
 (segment (start 203.808124 41.487) (end 206.33906 41.487) (width 0.2) (layer "F.Cu") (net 3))
 (segment (start 217.0525 64.1125) (end 217.52 64.58) (width 0.2) (layer "F.Cu") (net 3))
 (segment (start 205.89875 45.09) (end 205.285124 45.09) (width 0.2) (layer "F.Cu") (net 3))
 (segment (start 218.023669 71.7115) (end 217.322669 72.4125) (width 0.2) (layer "F.Cu") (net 3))
 (segment (start 216.35 70.25) (end 216.6115 70.5115) (width 0.2) (layer "F.Cu") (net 3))
 (segment (start 206.33906 41.487) (end 218.38 53.52794) (width 0.2) (layer "F.Cu") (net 3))
 (segment (start 216.6115 70.5115) (end 218.08 70.5115) (width 0.2) (layer "F.Cu") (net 3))
 (segment (start 203.54675 41.748374) (end 203.808124 41.487) (width 0.2) (layer "F.Cu") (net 3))
 (segment (start 205.285124 45.09) (end 203.54675 43.351626) (width 0.2) (layer "F.Cu") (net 3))
 (segment (start 203.54675 43.351626) (end 203.54675 41.748374) (width 0.2) (layer "F.Cu") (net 3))
 (segment (start 215.10625 68.2625) (end 216.35 69.50625) (width 0.2) (layer "F.Cu") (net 3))
 (segment (start 216.35 69.50625) (end 216.35 70.25) (width 0.2) (layer "F.Cu") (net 3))
 (segment (start 217.322669 72.4125) (end 215.10625 72.4125) (width 0.2) (layer "F.Cu") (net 3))
 (segment (start 215.10625 72.4125) (end 215.10625 76.5625) (width 0.2) (layer "F.Cu") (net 3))
 (via (at 218.023669 71.7115) (size 0.6) (drill 0.3) (layers "F.Cu" "B.Cu") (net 3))
 (via (at 217.52 64.58) (size 0.6) (drill 0.3) (layers "F.Cu" "B.Cu") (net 3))
 (via (at 218.08 70.5115) (size 0.6) (drill 0.3) (layers "F.Cu" "B.Cu") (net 3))
 (via (at 218.38 57.31) (size 0.6) (drill 0.3) (layers "F.Cu" "B.Cu") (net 3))
 (segment (start 218.0115 71.7115) (end 218.023669 71.7115) (width 0.2) (layer "B.Cu") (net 3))
 (segment (start 215.10625 60.74375) (end 215.10625 64.1125) (width 0.2) (layer "B.Cu") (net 3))
 (segment (start 218.08 71.5) (end 217.94 71.64) (width 0.2) (layer "B.Cu") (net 3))
 (segment (start 218.38 57.47) (end 215.10625 60.74375) (width 0.2) (layer "B.Cu") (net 3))
 (segment (start 218.38 57.31) (end 218.38 57.47) (width 0.2) (layer "B.Cu") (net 3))
 (segment (start 217.52 64.58) (end 215.10625 66.99375) (width 0.2) (layer "B.Cu") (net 3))
 (segment (start 215.10625 66.99375) (end 215.10625 68.2625) (width 0.2) (layer "B.Cu") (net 3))
 (segment (start 217.94 71.64) (end 218.0115 71.7115) (width 0.2) (layer "B.Cu") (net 3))
 (segment (start 218.08 70.5115) (end 218.08 71.5) (width 0.2) (layer "B.Cu") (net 3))
 (segment (start 142.129814 63.369) (end 203.59409 63.369) (width 0.2) (layer "F.Cu") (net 9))
 (segment (start 218.8165 65.48225) (end 220.18625 64.1125) (width 0.2) (layer "F.Cu") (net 9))
 (segment (start 138.188814 67.31) (end 142.129814 63.369) (width 0.2) (layer "F.Cu") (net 9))
 (segment (start 132.3975 67.31) (end 138.188814 67.31) (width 0.2) (layer "F.Cu") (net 9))
 (segment (start 203.59409 63.369) (end 205.70734 65.48225) (width 0.2) (layer "F.Cu") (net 9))
 (segment (start 205.70734 65.48225) (end 218.8165 65.48225) (width 0.2) (layer "F.Cu") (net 9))
 (segment (start 168.516186 67.31) (end 169.917186 65.909) (width 0.2) (layer "F.Cu") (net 2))
 (segment (start 176.726186 66.63) (end 188.246186 66.63) (width 0.2) (layer "F.Cu") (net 2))
 (segment (start 196.107686 66.9615) (end 218.88525 66.9615) (width 0.2) (layer "F.Cu") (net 2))
 (segment (start 195.055186 65.909) (end 196.107686 66.9615) (width 0.2) (layer "F.Cu") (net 2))
 (segment (start 188.967186 65.909) (end 195.055186 65.909) (width 0.2) (layer "F.Cu") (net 2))
 (segment (start 188.246186 66.63) (end 188.967186 65.909) (width 0.2) (layer "F.Cu") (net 2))
 (segment (start 218.88525 66.9615) (end 220.18625 68.2625) (width 0.2) (layer "F.Cu") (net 2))
 (segment (start 176.005186 65.909) (end 176.726186 66.63) (width 0.2) (layer "F.Cu") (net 2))
 (segment (start 169.917186 65.909) (end 176.005186 65.909) (width 0.2) (layer "F.Cu") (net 2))
 (segment (start 151.4475 67.31) (end 168.516186 67.31) (width 0.2) (layer "F.Cu") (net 2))
 (segment (start 190.902684 68.98) (end 192.383684 67.499) (width 0.2) (layer "F.Cu") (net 21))
 (segment (start 218.88525 71.1115) (end 220.18625 72.4125) (width 0.2) (layer "F.Cu") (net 21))
 (segment (start 203.57409 67.499) (end 207.18659 71.1115) (width 0.2) (layer "F.Cu") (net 21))
 (segment (start 189.236186 68.98) (end 190.902684 68.98) (width 0.2) (layer "F.Cu") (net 21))
 (segment (start 192.383684 67.499) (end 203.57409 67.499) (width 0.2) (layer "F.Cu") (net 21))
 (segment (start 187.566186 67.31) (end 189.236186 68.98) (width 0.2) (layer "F.Cu") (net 21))
 (segment (start 207.18659 71.1115) (end 218.88525 71.1115) (width 0.2) (layer "F.Cu") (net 21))
 (segment (start 170.4975 67.31) (end 187.566186 67.31) (width 0.2) (layer "F.Cu") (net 21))
 (segment (start 190.1175 66.74) (end 194.77 66.74) (width 0.2) (layer "F.Cu") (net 4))
 (segment (start 189.5475 67.31) (end 190.1175 66.74) (width 0.2) (layer "F.Cu") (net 4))
 (via (at 194.77 66.74) (size 0.6) (drill 0.3) (layers "F.Cu" "B.Cu") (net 4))
 (segment (start 194.77 66.74) (end 194.77 67.92) (width 0.2) (layer "B.Cu") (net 4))
 (segment (start 194.77 67.92) (end 204.78225 77.93225) (width 0.2) (layer "B.Cu") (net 4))
 (segment (start 204.78225 77.93225) (end 218.8165 77.93225) (width 0.2) (layer "B.Cu") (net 4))
 (segment (start 218.8165 77.93225) (end 220.18625 76.5625) (width 0.2) (layer "B.Cu") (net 4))
 (segment (start 157.566186 47.47) (end 169.306186 47.47) (width 0.2) (layer "F.Cu") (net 7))
 (segment (start 138.7475 45.72) (end 132.956186 45.72) (width 0.2) (layer "F.Cu") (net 7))
 (segment (start 177.947186 46.859) (end 195.055186 46.859) (width 0.2) (layer "F.Cu") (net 7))
 (segment (start 169.917186 46.859) (end 176.005186 46.859) (width 0.2) (layer "F.Cu") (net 7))
 (segment (start 169.306186 47.47) (end 169.917186 46.859) (width 0.2) (layer "F.Cu") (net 7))
 (segment (start 195.055186 46.859) (end 195.826186 47.63) (width 0.2) (layer "F.Cu") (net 7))
 (segment (start 155.816186 45.72) (end 157.566186 47.47) (width 0.2) (layer "F.Cu") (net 7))
 (segment (start 138.7475 45.72) (end 155.816186 45.72) (width 0.2) (layer "F.Cu") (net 7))
 (segment (start 132.956186 45.72) (end 130.9965 47.679686) (width 0.2) (layer "F.Cu") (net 7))
 (segment (start 138.7475 56.72153) (end 138.7475 64.77) (width 0.2) (layer "F.Cu") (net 7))
 (segment (start 130.9965 48.97053) (end 138.7475 56.72153) (width 0.2) (layer "F.Cu") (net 7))
 (segment (start 130.9965 47.679686) (end 130.9965 48.97053) (width 0.2) (layer "F.Cu") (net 7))
 (segment (start 195.826186 47.63) (end 205.89875 47.63) (width 0.2) (layer "F.Cu") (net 7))
 (segment (start 176.005186 46.859) (end 176.976186 47.83) (width 0.2) (layer "F.Cu") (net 7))
 (segment (start 176.976186 47.83) (end 177.947186 46.859) (width 0.2) (layer "F.Cu") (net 7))
 (segment (start 166.1 64.22) (end 166.16 64.16) (width 0.2) (layer "F.Cu") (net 1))
 (segment (start 159.5 64.77) (end 160.05 64.22) (width 0.2) (layer "F.Cu") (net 1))
 (segment (start 157.7975 64.77) (end 159.5 64.77) (width 0.2) (layer "F.Cu") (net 1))
 (segment (start 160.05 64.22) (end 166.1 64.22) (width 0.2) (layer "F.Cu") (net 1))
 (via (at 160.05 64.22) (size 0.6) (drill 0.3) (layers "F.Cu" "B.Cu") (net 1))
 (via (at 166.16 64.16) (size 0.6) (drill 0.3) (layers "F.Cu" "B.Cu") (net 1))
 (segment (start 155.219 45.750086) (end 157.051086 43.918) (width 0.2) (layer "B.Cu") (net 1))
 (segment (start 157.051086 43.918) (end 199.64675 43.918) (width 0.2) (layer "B.Cu") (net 1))
 (segment (start 155.219 48.078943) (end 155.219 45.750086) (width 0.2) (layer "B.Cu") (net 1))
 (segment (start 155.571057 48.431) (end 155.219 48.078943) (width 0.2) (layer "B.Cu") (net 1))
 (segment (start 166.16 50.76) (end 163.831 48.431) (width 0.2) (layer "B.Cu") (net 1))
 (segment (start 199.64675 43.918) (end 205.89875 50.17) (width 0.2) (layer "B.Cu") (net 1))
 (segment (start 166.16 64.16) (end 166.16 50.76) (width 0.2) (layer "B.Cu") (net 1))
 (segment (start 163.831 48.431) (end 155.571057 48.431) (width 0.2) (layer "B.Cu") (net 1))
 (segment (start 160.05 64.22) (end 157.7975 61.9675) (width 0.2) (layer "B.Cu") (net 1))
 (segment (start 157.7975 61.9675) (end 157.7975 45.72) (width 0.2) (layer "B.Cu") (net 1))
 (segment (start 207.386 46.166) (end 210.22 49) (width 0.2) (layer "F.Cu") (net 11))
 (segment (start 203.76 46.166) (end 207.386 46.166) (width 0.2) (layer "F.Cu") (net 11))
 (segment (start 176.8475 45.72) (end 178.74 45.72) (width 0.2) (layer "F.Cu") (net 11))
 (segment (start 178.2485 44.319) (end 201.913 44.319) (width 0.2) (layer "F.Cu") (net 11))
 (segment (start 178.74 45.72) (end 179.08 46.06) (width 0.2) (layer "F.Cu") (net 11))
 (segment (start 201.913 44.319) (end 203.76 46.166) (width 0.2) (layer "F.Cu") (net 11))
 (segment (start 176.8475 45.72) (end 178.2485 44.319) (width 0.2) (layer "F.Cu") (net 11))
 (via (at 210.22 49) (size 0.6) (drill 0.3) (layers "F.Cu" "B.Cu") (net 11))
 (via (at 179.08 46.06) (size 0.6) (drill 0.3) (layers "F.Cu" "B.Cu") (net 11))
 (segment (start 179.08 46.06) (end 180.5885 47.5685) (width 0.2) (layer "B.Cu") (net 11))
 (segment (start 210.22 49) (end 210.16 49.06) (width 0.2) (layer "B.Cu") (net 11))
 (segment (start 180.5885 61.029) (end 176.8475 64.77) (width 0.2) (layer "B.Cu") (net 11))
 (segment (start 210.16 49.06) (end 209.54875 49.06) (width 0.2) (layer "B.Cu") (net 11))
 (segment (start 209.54875 49.06) (end 205.89875 52.71) (width 0.2) (layer "B.Cu") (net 11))
 (segment (start 180.5885 47.5685) (end 180.5885 61.029) (width 0.2) (layer "B.Cu") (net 11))
 (segment (start 195.8975 45.72) (end 196.7445 46.567) (width 0.2) (layer "F.Cu") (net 12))
 (segment (start 221.48725 61.71519) (end 221.48725 64.651392) (width 0.2) (layer "F.Cu") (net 12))
 (segment (start 206.96175 54.187) (end 205.89875 55.25) (width 0.2) (layer "F.Cu") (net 12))
 (segment (start 206.33906 46.567) (end 221.48725 61.71519) (width 0.2) (layer "F.Cu") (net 12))
 (segment (start 201.5 64.77) (end 201.88 64.39) (width 0.2) (layer "F.Cu") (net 12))
 (segment (start 221.48725 64.651392) (end 220.255392 65.88325) (width 0.2) (layer "F.Cu") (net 12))
 (segment (start 206.96175 47.18969) (end 206.96175 54.187) (width 0.2) (layer "F.Cu") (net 12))
 (segment (start 220.255392 65.88325) (end 197.01075 65.88325) (width 0.2) (layer "F.Cu") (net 12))
 (segment (start 195.8975 64.77) (end 201.5 64.77) (width 0.2) (layer "F.Cu") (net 12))
 (segment (start 197.01075 65.88325) (end 195.8975 64.77) (width 0.2) (layer "F.Cu") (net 12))
 (segment (start 206.33906 46.567) (end 206.96175 47.18969) (width 0.2) (layer "F.Cu") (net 12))
 (segment (start 196.7445 46.567) (end 206.33906 46.567) (width 0.2) (layer "F.Cu") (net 12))
 (via (at 201.88 64.39) (size 0.6) (drill 0.3) (layers "F.Cu" "B.Cu") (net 12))
 (segment (start 201.88 58.1) (end 204.73 55.25) (width 0.2) (layer "B.Cu") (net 12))
 (segment (start 204.73 55.25) (end 205.89875 55.25) (width 0.2) (layer "B.Cu") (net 12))
 (segment (start 196.5325 64.77) (end 195.8975 64.77) (width 0.2) (layer "B.Cu") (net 12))
 (segment (start 201.88 64.39) (end 201.88 58.1) (width 0.2) (layer "B.Cu") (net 12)))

